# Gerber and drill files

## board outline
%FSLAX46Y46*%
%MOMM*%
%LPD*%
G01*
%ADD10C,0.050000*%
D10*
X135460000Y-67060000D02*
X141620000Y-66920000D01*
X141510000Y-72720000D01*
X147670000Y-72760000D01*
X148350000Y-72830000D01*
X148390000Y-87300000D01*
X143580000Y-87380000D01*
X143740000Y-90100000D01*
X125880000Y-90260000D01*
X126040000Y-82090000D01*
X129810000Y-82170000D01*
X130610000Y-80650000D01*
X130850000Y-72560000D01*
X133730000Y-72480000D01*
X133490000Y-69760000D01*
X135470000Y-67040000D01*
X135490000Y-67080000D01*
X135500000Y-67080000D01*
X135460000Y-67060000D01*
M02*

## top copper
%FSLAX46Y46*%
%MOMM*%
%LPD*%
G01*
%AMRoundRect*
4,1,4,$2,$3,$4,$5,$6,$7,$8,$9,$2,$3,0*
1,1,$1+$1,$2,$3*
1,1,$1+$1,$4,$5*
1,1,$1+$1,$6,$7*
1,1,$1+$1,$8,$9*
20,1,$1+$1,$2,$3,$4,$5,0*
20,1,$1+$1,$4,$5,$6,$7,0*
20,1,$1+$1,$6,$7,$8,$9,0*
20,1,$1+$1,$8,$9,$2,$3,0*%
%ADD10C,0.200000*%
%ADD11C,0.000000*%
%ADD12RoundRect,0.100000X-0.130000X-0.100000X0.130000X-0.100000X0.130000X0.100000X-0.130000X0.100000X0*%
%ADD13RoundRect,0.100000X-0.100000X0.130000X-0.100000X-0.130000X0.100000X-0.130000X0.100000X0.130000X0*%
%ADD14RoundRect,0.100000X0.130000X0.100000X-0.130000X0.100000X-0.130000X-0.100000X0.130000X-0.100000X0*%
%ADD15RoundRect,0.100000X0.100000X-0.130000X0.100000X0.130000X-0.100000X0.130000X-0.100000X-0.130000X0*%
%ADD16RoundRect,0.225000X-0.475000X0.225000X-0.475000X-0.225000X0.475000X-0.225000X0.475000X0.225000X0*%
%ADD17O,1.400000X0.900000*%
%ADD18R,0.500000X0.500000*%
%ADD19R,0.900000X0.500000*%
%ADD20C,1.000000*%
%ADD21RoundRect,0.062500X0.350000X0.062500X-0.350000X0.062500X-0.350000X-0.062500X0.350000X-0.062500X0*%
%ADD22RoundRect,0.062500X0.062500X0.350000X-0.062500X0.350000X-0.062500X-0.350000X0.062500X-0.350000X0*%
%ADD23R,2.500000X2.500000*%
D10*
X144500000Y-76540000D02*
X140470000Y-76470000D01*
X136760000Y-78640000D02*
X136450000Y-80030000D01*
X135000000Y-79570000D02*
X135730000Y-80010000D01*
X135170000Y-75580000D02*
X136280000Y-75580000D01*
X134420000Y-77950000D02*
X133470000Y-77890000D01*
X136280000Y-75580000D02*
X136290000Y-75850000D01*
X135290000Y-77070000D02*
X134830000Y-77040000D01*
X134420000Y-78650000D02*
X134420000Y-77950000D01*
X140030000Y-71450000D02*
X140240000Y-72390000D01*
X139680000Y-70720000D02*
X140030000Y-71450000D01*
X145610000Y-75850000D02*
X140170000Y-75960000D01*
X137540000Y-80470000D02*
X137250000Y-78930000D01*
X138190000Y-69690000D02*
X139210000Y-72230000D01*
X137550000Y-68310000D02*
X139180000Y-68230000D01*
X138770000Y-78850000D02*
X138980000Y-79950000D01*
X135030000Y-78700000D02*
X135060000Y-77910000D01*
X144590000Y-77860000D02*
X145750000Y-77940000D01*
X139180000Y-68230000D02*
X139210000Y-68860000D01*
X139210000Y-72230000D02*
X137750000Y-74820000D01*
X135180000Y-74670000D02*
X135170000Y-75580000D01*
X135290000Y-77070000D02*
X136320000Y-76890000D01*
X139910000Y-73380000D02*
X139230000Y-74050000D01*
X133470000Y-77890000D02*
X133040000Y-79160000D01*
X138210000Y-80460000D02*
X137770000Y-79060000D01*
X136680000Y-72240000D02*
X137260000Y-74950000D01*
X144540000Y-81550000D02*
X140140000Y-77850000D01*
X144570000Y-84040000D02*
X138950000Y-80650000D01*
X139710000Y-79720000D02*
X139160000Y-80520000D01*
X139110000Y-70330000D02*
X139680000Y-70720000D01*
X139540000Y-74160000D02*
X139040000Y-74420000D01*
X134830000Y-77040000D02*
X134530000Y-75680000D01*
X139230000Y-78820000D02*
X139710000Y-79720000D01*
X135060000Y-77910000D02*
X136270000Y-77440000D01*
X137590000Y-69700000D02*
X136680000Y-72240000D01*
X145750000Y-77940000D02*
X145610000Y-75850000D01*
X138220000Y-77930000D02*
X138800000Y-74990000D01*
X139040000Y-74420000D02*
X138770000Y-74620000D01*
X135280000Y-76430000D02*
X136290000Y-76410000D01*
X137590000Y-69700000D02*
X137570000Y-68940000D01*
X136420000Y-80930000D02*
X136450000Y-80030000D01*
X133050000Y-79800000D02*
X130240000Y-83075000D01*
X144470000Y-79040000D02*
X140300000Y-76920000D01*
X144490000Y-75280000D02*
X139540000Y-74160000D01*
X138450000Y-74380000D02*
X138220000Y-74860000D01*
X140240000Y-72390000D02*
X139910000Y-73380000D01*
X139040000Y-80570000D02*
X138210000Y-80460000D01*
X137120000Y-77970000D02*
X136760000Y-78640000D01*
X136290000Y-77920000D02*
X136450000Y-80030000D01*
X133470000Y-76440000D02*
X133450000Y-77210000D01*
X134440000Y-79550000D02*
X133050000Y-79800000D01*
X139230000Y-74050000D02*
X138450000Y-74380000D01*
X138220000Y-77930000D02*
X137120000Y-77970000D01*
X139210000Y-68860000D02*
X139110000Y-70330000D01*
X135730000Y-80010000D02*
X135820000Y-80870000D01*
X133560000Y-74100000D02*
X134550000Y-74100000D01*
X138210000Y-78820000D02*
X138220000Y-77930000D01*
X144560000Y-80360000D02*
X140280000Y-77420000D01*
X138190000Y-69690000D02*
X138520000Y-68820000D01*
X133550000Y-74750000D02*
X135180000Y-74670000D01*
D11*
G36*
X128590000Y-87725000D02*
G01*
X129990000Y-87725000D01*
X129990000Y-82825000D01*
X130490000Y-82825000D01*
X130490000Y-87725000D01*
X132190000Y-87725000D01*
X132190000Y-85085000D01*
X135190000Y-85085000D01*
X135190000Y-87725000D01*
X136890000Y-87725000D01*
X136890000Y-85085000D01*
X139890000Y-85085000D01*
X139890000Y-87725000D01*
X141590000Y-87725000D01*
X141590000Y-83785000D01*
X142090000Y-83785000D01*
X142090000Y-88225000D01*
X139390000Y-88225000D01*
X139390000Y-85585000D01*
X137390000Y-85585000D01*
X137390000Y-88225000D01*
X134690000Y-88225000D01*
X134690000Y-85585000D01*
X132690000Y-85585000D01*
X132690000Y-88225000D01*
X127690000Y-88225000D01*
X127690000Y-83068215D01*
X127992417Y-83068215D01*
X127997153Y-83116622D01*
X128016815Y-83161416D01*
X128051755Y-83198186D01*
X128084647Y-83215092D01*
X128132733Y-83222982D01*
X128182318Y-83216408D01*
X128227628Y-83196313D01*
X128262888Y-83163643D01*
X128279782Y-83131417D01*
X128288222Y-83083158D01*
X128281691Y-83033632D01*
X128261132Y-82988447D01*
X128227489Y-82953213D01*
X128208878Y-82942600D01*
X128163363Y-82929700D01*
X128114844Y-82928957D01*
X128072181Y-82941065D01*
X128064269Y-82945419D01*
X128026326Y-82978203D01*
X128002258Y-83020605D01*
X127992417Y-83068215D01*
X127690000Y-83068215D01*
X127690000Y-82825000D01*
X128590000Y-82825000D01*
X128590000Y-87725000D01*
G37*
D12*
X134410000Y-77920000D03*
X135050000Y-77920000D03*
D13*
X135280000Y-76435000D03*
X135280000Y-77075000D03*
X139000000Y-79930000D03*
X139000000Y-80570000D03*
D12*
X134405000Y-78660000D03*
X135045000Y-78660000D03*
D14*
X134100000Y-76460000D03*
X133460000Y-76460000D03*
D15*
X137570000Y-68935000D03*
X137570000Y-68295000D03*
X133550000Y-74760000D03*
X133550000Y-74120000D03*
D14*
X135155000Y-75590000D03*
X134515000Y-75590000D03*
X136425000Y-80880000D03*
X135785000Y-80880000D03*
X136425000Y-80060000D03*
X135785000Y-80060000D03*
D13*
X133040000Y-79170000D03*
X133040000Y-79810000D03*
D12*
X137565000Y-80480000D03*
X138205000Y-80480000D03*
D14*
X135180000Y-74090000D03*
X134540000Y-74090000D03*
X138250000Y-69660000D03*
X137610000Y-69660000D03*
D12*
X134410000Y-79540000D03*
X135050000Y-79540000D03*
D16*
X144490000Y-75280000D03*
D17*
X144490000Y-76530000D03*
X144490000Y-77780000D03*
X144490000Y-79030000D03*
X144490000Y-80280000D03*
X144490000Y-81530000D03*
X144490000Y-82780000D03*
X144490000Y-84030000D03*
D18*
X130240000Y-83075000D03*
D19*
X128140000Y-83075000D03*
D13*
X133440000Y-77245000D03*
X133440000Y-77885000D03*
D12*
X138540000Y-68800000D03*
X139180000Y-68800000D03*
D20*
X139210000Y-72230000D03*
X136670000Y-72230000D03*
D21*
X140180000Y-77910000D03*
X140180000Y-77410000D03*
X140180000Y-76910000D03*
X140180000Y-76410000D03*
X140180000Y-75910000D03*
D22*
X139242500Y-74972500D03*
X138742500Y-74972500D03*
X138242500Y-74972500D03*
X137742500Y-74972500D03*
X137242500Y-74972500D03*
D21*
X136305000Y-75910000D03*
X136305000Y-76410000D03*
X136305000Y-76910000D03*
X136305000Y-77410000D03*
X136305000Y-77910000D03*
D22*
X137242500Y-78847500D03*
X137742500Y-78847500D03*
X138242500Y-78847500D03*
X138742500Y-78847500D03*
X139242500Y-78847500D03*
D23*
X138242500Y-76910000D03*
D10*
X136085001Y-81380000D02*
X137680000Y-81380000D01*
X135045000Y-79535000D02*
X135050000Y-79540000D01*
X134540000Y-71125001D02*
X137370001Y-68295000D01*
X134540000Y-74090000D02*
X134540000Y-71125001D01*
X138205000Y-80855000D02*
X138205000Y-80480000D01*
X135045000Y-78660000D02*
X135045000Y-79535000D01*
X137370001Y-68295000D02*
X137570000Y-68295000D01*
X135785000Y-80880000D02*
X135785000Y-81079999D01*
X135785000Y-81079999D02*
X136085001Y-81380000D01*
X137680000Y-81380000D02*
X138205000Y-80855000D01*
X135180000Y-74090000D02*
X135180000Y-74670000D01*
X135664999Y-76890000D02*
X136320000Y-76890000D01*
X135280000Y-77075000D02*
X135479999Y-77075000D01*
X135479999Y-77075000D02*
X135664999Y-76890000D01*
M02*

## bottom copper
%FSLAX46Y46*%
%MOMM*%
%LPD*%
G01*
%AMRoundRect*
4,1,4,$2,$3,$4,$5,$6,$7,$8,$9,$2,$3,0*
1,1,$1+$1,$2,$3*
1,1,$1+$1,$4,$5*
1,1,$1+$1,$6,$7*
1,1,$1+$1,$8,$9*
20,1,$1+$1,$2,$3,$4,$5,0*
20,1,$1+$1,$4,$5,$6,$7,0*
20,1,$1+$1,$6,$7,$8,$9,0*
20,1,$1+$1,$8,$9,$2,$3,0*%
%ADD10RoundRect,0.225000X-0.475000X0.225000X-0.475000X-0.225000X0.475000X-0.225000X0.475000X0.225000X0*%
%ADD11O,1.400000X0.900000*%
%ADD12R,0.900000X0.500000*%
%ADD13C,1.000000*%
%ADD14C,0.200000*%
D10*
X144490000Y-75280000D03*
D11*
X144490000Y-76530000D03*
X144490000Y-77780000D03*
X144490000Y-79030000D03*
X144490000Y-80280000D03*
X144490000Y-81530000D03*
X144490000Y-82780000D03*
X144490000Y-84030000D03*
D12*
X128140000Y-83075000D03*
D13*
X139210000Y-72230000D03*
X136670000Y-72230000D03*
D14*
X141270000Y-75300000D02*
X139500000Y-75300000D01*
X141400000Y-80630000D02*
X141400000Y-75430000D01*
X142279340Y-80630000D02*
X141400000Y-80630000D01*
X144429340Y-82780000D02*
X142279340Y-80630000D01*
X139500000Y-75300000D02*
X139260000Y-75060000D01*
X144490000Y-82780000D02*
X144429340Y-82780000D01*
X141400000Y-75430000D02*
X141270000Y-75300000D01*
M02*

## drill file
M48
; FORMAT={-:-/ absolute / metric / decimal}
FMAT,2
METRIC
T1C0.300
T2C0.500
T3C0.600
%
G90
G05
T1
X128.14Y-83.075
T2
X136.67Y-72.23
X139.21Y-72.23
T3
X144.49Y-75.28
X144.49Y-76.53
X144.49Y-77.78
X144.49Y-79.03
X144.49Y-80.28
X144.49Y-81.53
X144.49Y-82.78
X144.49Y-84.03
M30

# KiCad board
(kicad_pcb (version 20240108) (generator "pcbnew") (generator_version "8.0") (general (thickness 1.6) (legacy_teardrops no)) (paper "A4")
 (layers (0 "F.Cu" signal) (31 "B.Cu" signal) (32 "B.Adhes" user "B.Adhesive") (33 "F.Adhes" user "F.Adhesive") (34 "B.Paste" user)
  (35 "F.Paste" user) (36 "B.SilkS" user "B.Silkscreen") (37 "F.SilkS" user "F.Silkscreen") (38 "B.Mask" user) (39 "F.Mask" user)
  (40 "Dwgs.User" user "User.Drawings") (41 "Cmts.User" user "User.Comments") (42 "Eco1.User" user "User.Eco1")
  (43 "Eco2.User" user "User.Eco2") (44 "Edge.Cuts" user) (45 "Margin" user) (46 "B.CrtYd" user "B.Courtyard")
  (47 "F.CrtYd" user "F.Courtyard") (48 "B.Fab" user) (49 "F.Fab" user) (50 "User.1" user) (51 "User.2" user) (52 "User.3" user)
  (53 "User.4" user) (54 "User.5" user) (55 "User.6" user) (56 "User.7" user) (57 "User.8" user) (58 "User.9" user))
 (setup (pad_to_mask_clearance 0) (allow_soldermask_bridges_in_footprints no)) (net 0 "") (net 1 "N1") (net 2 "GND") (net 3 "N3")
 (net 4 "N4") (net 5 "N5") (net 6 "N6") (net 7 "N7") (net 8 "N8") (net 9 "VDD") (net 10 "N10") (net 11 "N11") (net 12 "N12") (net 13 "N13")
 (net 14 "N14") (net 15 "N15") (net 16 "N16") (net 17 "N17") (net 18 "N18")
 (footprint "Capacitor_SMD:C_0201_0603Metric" (layer "F.Cu") (at 134.73 77.92)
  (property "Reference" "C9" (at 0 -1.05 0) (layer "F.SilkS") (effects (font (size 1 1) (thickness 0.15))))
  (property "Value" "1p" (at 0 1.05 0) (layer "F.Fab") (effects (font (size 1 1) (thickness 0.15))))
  (pad "" smd roundrect (at -0.345 0) (size 0.318 0.36) (layers "F.Paste") (roundrect_rratio 0.25))
  (pad "" smd roundrect (at 0.345 0) (size 0.318 0.36) (layers "F.Paste") (roundrect_rratio 0.25))
  (pad "1" smd roundrect (at -0.32 0) (size 0.46 0.4) (layers "F.Cu" "F.Mask") (roundrect_rratio 0.25) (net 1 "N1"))
  (pad "2" smd roundrect (at 0.32 0) (size 0.46 0.4) (layers "F.Cu" "F.Mask") (roundrect_rratio 0.25) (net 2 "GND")))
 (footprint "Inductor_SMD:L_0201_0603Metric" (layer "F.Cu") (at 135.28 76.755 -90)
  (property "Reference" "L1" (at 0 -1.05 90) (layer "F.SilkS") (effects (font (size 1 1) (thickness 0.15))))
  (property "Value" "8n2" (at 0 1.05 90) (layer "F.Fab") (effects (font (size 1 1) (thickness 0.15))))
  (pad "" smd roundrect (at -0.345 0 270) (size 0.318 0.36) (layers "F.Paste") (roundrect_rratio 0.25))
  (pad "" smd roundrect (at 0.345 0 270) (size 0.318 0.36) (layers "F.Paste") (roundrect_rratio 0.25))
  (pad "1" smd roundrect (at -0.32 0 270) (size 0.46 0.4) (layers "F.Cu" "F.Mask") (roundrect_rratio 0.25) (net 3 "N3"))
  (pad "2" smd roundrect (at 0.32 0 270) (size 0.46 0.4) (layers "F.Cu" "F.Mask") (roundrect_rratio 0.25) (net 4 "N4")))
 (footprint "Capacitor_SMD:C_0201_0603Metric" (layer "F.Cu") (at 139 80.25 -90)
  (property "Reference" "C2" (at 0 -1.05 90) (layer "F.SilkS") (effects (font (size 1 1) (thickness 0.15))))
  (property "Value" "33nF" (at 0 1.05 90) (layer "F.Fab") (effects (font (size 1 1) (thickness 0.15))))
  (pad "" smd roundrect (at -0.345 0 270) (size 0.318 0.36) (layers "F.Paste") (roundrect_rratio 0.25))
  (pad "" smd roundrect (at 0.345 0 270) (size 0.318 0.36) (layers "F.Paste") (roundrect_rratio 0.25))
  (pad "1" smd roundrect (at -0.32 0 270) (size 0.46 0.4) (layers "F.Cu" "F.Mask") (roundrect_rratio 0.25) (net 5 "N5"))
  (pad "2" smd roundrect (at 0.32 0 270) (size 0.46 0.4) (layers "F.Cu" "F.Mask") (roundrect_rratio 0.25) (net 2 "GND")))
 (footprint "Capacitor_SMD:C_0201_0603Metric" (layer "F.Cu") (at 134.725 78.66)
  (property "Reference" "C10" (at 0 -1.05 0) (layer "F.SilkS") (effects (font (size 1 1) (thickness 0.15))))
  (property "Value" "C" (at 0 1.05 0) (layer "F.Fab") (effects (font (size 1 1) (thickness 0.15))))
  (pad "" smd roundrect (at -0.345 0) (size 0.318 0.36) (layers "F.Paste") (roundrect_rratio 0.25))
  (pad "" smd roundrect (at 0.345 0) (size 0.318 0.36) (layers "F.Paste") (roundrect_rratio 0.25))
  (pad "1" smd roundrect (at -0.32 0) (size 0.46 0.4) (layers "F.Cu" "F.Mask") (roundrect_rratio 0.25) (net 1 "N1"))
  (pad "2" smd roundrect (at 0.32 0) (size 0.46 0.4) (layers "F.Cu" "F.Mask") (roundrect_rratio 0.25) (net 2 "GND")))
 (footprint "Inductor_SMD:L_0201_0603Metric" (layer "F.Cu") (at 133.78 76.46 180)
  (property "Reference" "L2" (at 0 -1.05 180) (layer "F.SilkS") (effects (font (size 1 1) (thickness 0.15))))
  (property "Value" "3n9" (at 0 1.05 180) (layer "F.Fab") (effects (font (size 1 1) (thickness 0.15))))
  (pad "" smd roundrect (at -0.345 0 180) (size 0.318 0.36) (layers "F.Paste") (roundrect_rratio 0.25))
  (pad "" smd roundrect (at 0.345 0 180) (size 0.318 0.36) (layers "F.Paste") (roundrect_rratio 0.25))
  (pad "1" smd roundrect (at -0.32 0 180) (size 0.46 0.4) (layers "F.Cu" "F.Mask") (roundrect_rratio 0.25) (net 3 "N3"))
  (pad "2" smd roundrect (at 0.32 0 180) (size 0.46 0.4) (layers "F.Cu" "F.Mask") (roundrect_rratio 0.25) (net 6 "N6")))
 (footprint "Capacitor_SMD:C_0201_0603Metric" (layer "F.Cu") (at 137.57 68.615 90)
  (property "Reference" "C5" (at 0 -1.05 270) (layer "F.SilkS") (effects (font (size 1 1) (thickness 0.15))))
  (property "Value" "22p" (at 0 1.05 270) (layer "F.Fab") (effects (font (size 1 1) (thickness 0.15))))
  (pad "" smd roundrect (at -0.345 0 90) (size 0.318 0.36) (layers "F.Paste") (roundrect_rratio 0.25))
  (pad "" smd roundrect (at 0.345 0 90) (size 0.318 0.36) (layers "F.Paste") (roundrect_rratio 0.25))
  (pad "1" smd roundrect (at -0.32 0 90) (size 0.46 0.4) (layers "F.Cu" "F.Mask") (roundrect_rratio 0.25) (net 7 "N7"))
  (pad "2" smd roundrect (at 0.32 0 90) (size 0.46 0.4) (layers "F.Cu" "F.Mask") (roundrect_rratio 0.25) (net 2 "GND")))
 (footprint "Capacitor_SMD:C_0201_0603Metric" (layer "F.Cu") (at 133.55 74.44 90)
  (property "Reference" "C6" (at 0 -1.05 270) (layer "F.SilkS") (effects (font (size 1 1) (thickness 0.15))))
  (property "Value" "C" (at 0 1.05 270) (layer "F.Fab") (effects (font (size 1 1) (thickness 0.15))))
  (pad "" smd roundrect (at -0.345 0 90) (size 0.318 0.36) (layers "F.Paste") (roundrect_rratio 0.25))
  (pad "" smd roundrect (at 0.345 0 90) (size 0.318 0.36) (layers "F.Paste") (roundrect_rratio 0.25))
  (pad "1" smd roundrect (at -0.32 0 90) (size 0.46 0.4) (layers "F.Cu" "F.Mask") (roundrect_rratio 0.25) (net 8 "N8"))
  (pad "2" smd roundrect (at 0.32 0 90) (size 0.46 0.4) (layers "F.Cu" "F.Mask") (roundrect_rratio 0.25) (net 2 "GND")))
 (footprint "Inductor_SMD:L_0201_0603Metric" (layer "F.Cu") (at 134.835 75.59 180)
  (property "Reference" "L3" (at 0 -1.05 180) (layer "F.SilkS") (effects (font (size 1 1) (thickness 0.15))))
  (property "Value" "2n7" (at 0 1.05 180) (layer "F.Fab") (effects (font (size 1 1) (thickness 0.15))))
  (pad "" smd roundrect (at -0.345 0 180) (size 0.318 0.36) (layers "F.Paste") (roundrect_rratio 0.25))
  (pad "" smd roundrect (at 0.345 0 180) (size 0.318 0.36) (layers "F.Paste") (roundrect_rratio 0.25))
  (pad "1" smd roundrect (at -0.32 0 180) (size 0.46 0.4) (layers "F.Cu" "F.Mask") (roundrect_rratio 0.25) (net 8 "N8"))
  (pad "2" smd roundrect (at 0.32 0 180) (size 0.46 0.4) (layers "F.Cu" "F.Mask") (roundrect_rratio 0.25) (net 4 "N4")))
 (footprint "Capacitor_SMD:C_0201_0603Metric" (layer "F.Cu") (at 136.105 80.88 180)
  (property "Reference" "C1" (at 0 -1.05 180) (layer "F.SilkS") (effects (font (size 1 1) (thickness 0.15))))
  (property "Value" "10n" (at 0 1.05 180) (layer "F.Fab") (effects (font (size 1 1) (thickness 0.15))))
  (pad "" smd roundrect (at -0.345 0 180) (size 0.318 0.36) (layers "F.Paste") (roundrect_rratio 0.25))
  (pad "" smd roundrect (at 0.345 0 180) (size 0.318 0.36) (layers "F.Paste") (roundrect_rratio 0.25))
  (pad "1" smd roundrect (at -0.32 0 180) (size 0.46 0.4) (layers "F.Cu" "F.Mask") (roundrect_rratio 0.25) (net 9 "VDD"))
  (pad "2" smd roundrect (at 0.32 0 180) (size 0.46 0.4) (layers "F.Cu" "F.Mask") (roundrect_rratio 0.25) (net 2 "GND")))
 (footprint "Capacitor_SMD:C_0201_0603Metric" (layer "F.Cu") (at 136.105 80.06 180)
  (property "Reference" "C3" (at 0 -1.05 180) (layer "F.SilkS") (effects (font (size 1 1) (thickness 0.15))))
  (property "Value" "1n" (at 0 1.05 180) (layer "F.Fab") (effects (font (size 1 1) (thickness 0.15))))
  (pad "" smd roundrect (at -0.345 0 180) (size 0.318 0.36) (layers "F.Paste") (roundrect_rratio 0.25))
  (pad "" smd roundrect (at 0.345 0 180) (size 0.318 0.36) (layers "F.Paste") (roundrect_rratio 0.25))
  (pad "1" smd roundrect (at -0.32 0 180) (size 0.46 0.4) (layers "F.Cu" "F.Mask") (roundrect_rratio 0.25) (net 9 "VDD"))
  (pad "2" smd roundrect (at 0.32 0 180) (size 0.46 0.4) (layers "F.Cu" "F.Mask") (roundrect_rratio 0.25) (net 2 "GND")))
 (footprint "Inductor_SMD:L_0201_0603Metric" (layer "F.Cu") (at 133.04 79.49 -90)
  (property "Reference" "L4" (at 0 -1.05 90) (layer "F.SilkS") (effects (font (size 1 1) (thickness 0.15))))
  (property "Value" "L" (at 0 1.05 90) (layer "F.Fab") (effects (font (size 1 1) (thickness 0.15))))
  (pad "" smd roundrect (at -0.345 0 270) (size 0.318 0.36) (layers "F.Paste") (roundrect_rratio 0.25))
  (pad "" smd roundrect (at 0.345 0 270) (size 0.318 0.36) (layers "F.Paste") (roundrect_rratio 0.25))
  (pad "1" smd roundrect (at -0.32 0 270) (size 0.46 0.4) (layers "F.Cu" "F.Mask") (roundrect_rratio 0.25) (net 1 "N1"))
  (pad "2" smd roundrect (at 0.32 0 270) (size 0.46 0.4) (layers "F.Cu" "F.Mask") (roundrect_rratio 0.25) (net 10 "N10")))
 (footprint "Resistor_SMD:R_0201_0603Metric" (layer "F.Cu") (at 137.885 80.48)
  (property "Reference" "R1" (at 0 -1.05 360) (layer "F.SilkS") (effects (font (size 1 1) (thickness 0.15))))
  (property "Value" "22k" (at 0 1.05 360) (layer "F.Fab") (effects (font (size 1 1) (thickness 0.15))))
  (pad "" smd roundrect (at -0.345 0) (size 0.318 0.36) (layers "F.Paste") (roundrect_rratio 0.25))
  (pad "" smd roundrect (at 0.345 0) (size 0.318 0.36) (layers "F.Paste") (roundrect_rratio 0.25))
  (pad "1" smd roundrect (at -0.32 0) (size 0.46 0.4) (layers "F.Cu" "F.Mask") (roundrect_rratio 0.25) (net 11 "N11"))
  (pad "2" smd roundrect (at 0.32 0) (size 0.46 0.4) (layers "F.Cu" "F.Mask") (roundrect_rratio 0.25) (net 2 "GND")))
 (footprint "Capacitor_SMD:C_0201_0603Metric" (layer "F.Cu") (at 134.86 74.09 180)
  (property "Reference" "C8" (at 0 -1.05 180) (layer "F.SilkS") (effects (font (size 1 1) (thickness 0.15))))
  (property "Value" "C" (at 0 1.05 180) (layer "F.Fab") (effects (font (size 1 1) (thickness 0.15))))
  (pad "" smd roundrect (at -0.345 0 180) (size 0.318 0.36) (layers "F.Paste") (roundrect_rratio 0.25))
  (pad "" smd roundrect (at 0.345 0 180) (size 0.318 0.36) (layers "F.Paste") (roundrect_rratio 0.25))
  (pad "1" smd roundrect (at -0.32 0 180) (size 0.46 0.4) (layers "F.Cu" "F.Mask") (roundrect_rratio 0.25) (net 8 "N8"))
  (pad "2" smd roundrect (at 0.32 0 180) (size 0.46 0.4) (layers "F.Cu" "F.Mask") (roundrect_rratio 0.25) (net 2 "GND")))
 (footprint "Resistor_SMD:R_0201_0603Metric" (layer "F.Cu") (at 137.93 69.66 180)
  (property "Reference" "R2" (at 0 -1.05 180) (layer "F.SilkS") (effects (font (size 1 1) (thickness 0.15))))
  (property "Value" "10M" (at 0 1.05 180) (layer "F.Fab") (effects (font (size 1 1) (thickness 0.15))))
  (pad "" smd roundrect (at -0.345 0 180) (size 0.318 0.36) (layers "F.Paste") (roundrect_rratio 0.25))
  (pad "" smd roundrect (at 0.345 0 180) (size 0.318 0.36) (layers "F.Paste") (roundrect_rratio 0.25))
  (pad "1" smd roundrect (at -0.32 0 180) (size 0.46 0.4) (layers "F.Cu" "F.Mask") (roundrect_rratio 0.25) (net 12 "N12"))
  (pad "2" smd roundrect (at 0.32 0 180) (size 0.46 0.4) (layers "F.Cu" "F.Mask") (roundrect_rratio 0.25) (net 7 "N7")))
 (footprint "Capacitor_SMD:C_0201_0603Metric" (layer "F.Cu") (at 134.73 79.54)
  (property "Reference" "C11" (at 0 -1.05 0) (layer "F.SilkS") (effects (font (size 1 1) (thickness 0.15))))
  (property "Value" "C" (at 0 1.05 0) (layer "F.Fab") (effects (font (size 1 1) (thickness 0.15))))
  (pad "" smd roundrect (at -0.345 0) (size 0.318 0.36) (layers "F.Paste") (roundrect_rratio 0.25))
  (pad "" smd roundrect (at 0.345 0) (size 0.318 0.36) (layers "F.Paste") (roundrect_rratio 0.25))
  (pad "1" smd roundrect (at -0.32 0) (size 0.46 0.4) (layers "F.Cu" "F.Mask") (roundrect_rratio 0.25) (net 10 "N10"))
  (pad "2" smd roundrect (at 0.32 0) (size 0.46 0.4) (layers "F.Cu" "F.Mask") (roundrect_rratio 0.25) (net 2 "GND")))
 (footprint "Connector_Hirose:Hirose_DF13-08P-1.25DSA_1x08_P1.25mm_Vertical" (layer "F.Cu") (at 144.49 75.28 -90)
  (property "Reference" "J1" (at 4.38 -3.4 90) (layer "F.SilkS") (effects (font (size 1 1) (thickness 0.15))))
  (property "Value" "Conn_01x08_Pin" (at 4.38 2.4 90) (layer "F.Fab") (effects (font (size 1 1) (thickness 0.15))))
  (pad "1" thru_hole roundrect (at 0 0 270) (size 0.9 1.4) (drill 0.6) (layers "*.Cu" "*.Mask") (remove_unused_layers no)
   (roundrect_rratio 0.25) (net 9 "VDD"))
  (pad "2" thru_hole oval (at 1.25 0 270) (size 0.9 1.4) (drill 0.6) (layers "*.Cu" "*.Mask") (remove_unused_layers no) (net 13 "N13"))
  (pad "3" thru_hole oval (at 2.5 0 270) (size 0.9 1.4) (drill 0.6) (layers "*.Cu" "*.Mask") (remove_unused_layers no) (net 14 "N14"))
  (pad "4" thru_hole oval (at 3.75 0 270) (size 0.9 1.4) (drill 0.6) (layers "*.Cu" "*.Mask") (remove_unused_layers no) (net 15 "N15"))
  (pad "5" thru_hole oval (at 5 0 270) (size 0.9 1.4) (drill 0.6) (layers "*.Cu" "*.Mask") (remove_unused_layers no) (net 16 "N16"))
  (pad "6" thru_hole oval (at 6.25 0 270) (size 0.9 1.4) (drill 0.6) (layers "*.Cu" "*.Mask") (remove_unused_layers no) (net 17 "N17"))
  (pad "7" thru_hole oval (at 7.5 0 270) (size 0.9 1.4) (drill 0.6) (layers "*.Cu" "*.Mask") (remove_unused_layers no) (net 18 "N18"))
  (pad "8" thru_hole oval (at 8.75 0 270) (size 0.9 1.4) (drill 0.6) (layers "*.Cu" "*.Mask") (remove_unused_layers no) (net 2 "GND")))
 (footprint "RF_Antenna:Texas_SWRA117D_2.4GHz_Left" (layer "F.Cu") (at 130.24 83.075 180)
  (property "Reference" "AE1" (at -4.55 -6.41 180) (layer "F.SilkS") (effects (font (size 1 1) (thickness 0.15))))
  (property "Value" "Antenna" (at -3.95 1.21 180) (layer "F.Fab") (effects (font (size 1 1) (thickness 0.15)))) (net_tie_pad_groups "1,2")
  (fp_poly
   (pts (xy -2.45 -2.51) (xy -4.45 -2.51) (xy -4.45 -5.15) (xy -7.15 -5.15) (xy -7.15 -2.51) (xy -9.15 -2.51) (xy -9.15 -5.15)
    (xy -11.85 -5.15) (xy -11.85 -0.71) (xy -11.35 -0.71) (xy -11.35 -4.65) (xy -9.65 -4.65) (xy -9.65 -2.01) (xy -6.65 -2.01)
    (xy -6.65 -4.65) (xy -4.95 -4.65) (xy -4.95 -2.01) (xy -1.95 -2.01) (xy -1.95 -4.65) (xy -0.25 -4.65) (xy -0.25 0.25) (xy 0.25 0.25)
    (xy 0.25 -4.65) (xy 1.65 -4.65) (xy 1.65 0.25) (xy 2.55 0.25) (xy 2.55 0.006785) (xy 2.247583 0.006785) (xy 2.237742 0.054395)
    (xy 2.213674 0.096797) (xy 2.175731 0.129581) (xy 2.167819 0.133935) (xy 2.125156 0.146043) (xy 2.076637 0.1453) (xy 2.031122 0.1324)
    (xy 2.012511 0.121787) (xy 1.978868 0.086553) (xy 1.958309 0.041368) (xy 1.951778 -0.008158) (xy 1.960218 -0.056417)
    (xy 1.977112 -0.088643) (xy 2.012372 -0.121313) (xy 2.057682 -0.141408) (xy 2.107267 -0.147982) (xy 2.155353 -0.140092)
    (xy 2.188245 -0.123186) (xy 2.223185 -0.086416) (xy 2.242847 -0.041622) (xy 2.247583 0.006785) (xy 2.55 0.006785) (xy 2.55 -5.15)
    (xy -2.45 -5.15) (xy -2.45 -2.51))
   (stroke (width 0) (type solid)) (fill solid) (layer "F.Cu"))
  (pad "1" connect rect (at 0 0 180) (size 0.5 0.5) (layers "F.Cu") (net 10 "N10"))
  (pad "2" thru_hole rect (at 2.1 0 180) (size 0.9 0.5) (drill 0.3) (layers "*.Cu") (remove_unused_layers no) (zone_connect 2)))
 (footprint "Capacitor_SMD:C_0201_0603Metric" (layer "F.Cu") (at 133.44 77.565 -90)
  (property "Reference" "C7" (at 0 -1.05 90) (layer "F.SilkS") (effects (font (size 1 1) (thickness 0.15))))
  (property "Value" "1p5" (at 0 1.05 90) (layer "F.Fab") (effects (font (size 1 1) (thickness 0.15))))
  (pad "" smd roundrect (at -0.345 0 270) (size 0.318 0.36) (layers "F.Paste") (roundrect_rratio 0.25))
  (pad "" smd roundrect (at 0.345 0 270) (size 0.318 0.36) (layers "F.Paste") (roundrect_rratio 0.25))
  (pad "1" smd roundrect (at -0.32 0 270) (size 0.46 0.4) (layers "F.Cu" "F.Mask") (roundrect_rratio 0.25) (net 6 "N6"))
  (pad "2" smd roundrect (at 0.32 0 270) (size 0.46 0.4) (layers "F.Cu" "F.Mask") (roundrect_rratio 0.25) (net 1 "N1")))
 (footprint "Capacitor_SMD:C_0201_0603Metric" (layer "F.Cu") (at 138.86 68.8)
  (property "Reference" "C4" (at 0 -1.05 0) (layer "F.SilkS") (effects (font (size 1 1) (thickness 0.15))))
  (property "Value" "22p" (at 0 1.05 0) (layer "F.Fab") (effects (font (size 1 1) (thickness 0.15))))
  (pad "" smd roundrect (at -0.345 0) (size 0.318 0.36) (layers "F.Paste") (roundrect_rratio 0.25))
  (pad "" smd roundrect (at 0.345 0) (size 0.318 0.36) (layers "F.Paste") (roundrect_rratio 0.25))
  (pad "1" smd roundrect (at -0.32 0) (size 0.46 0.4) (layers "F.Cu" "F.Mask") (roundrect_rratio 0.25) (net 12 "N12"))
  (pad "2" smd roundrect (at 0.32 0) (size 0.46 0.4) (layers "F.Cu" "F.Mask") (roundrect_rratio 0.25) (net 2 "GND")))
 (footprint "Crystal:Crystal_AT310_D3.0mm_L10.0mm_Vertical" (layer "F.Cu") (at 139.21 72.23 180)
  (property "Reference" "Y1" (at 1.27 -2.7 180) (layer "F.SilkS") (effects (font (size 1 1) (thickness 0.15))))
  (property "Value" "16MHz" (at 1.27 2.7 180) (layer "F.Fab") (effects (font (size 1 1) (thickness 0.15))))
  (pad "1" thru_hole circle (at 0 0 180) (size 1 1) (drill 0.5) (layers "*.Cu" "*.Mask") (remove_unused_layers no) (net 12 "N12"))
  (pad "2" thru_hole circle (at 2.54 0 180) (size 1 1) (drill 0.5) (layers "*.Cu" "*.Mask") (remove_unused_layers no) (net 7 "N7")))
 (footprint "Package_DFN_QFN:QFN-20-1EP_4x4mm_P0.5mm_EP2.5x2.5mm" (layer "F.Cu") (at 138.2425 76.91 180)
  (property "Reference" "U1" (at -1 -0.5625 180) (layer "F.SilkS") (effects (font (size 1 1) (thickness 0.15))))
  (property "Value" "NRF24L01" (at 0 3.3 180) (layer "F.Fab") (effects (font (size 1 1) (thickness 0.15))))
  (pad "" smd roundrect (at -0.625 -0.625 180) (size 1.01 1.01) (layers "F.Paste") (roundrect_rratio 0.247525))
  (pad "" smd roundrect (at -0.625 0.625 180) (size 1.01 1.01) (layers "F.Paste") (roundrect_rratio 0.247525))
  (pad "" smd roundrect (at 0.625 -0.625 180) (size 1.01 1.01) (layers "F.Paste") (roundrect_rratio 0.247525))
  (pad "" smd roundrect (at 0.625 0.625 180) (size 1.01 1.01) (layers "F.Paste") (roundrect_rratio 0.247525))
  (pad "1" smd roundrect (at -1.9375 -1 180) (size 0.825 0.25) (layers "F.Cu" "F.Paste" "F.Mask") (roundrect_rratio 0.25) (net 17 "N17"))
  (pad "2" smd roundrect (at -1.9375 -0.5 180) (size 0.825 0.25) (layers "F.Cu" "F.Paste" "F.Mask") (roundrect_rratio 0.25) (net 16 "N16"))
  (pad "3" smd roundrect (at -1.9375 0 180) (size 0.825 0.25) (layers "F.Cu" "F.Paste" "F.Mask") (roundrect_rratio 0.25) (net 15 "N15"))
  (pad "4" smd roundrect (at -1.9375 0.5 180) (size 0.825 0.25) (layers "F.Cu" "F.Paste" "F.Mask") (roundrect_rratio 0.25) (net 13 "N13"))
  (pad "5" smd roundrect (at -1.9375 1 180) (size 0.825 0.25) (layers "F.Cu" "F.Paste" "F.Mask") (roundrect_rratio 0.25) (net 14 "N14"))
  (pad "6" smd roundrect (at -1 1.9375 180) (size 0.25 0.825) (layers "F.Cu" "F.Paste" "F.Mask") (roundrect_rratio 0.25) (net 18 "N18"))
  (pad "7" smd roundrect (at -0.5 1.9375 180) (size 0.25 0.825) (layers "F.Cu" "F.Paste" "F.Mask") (roundrect_rratio 0.25) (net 9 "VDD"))
  (pad "8" smd roundrect (at 0 1.9375 180) (size 0.25 0.825) (layers "F.Cu" "F.Paste" "F.Mask") (roundrect_rratio 0.25) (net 2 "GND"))
  (pad "9" smd roundrect (at 0.5 1.9375 180) (size 0.25 0.825) (layers "F.Cu" "F.Paste" "F.Mask") (roundrect_rratio 0.25) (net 12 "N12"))
  (pad "10" smd roundrect (at 1 1.9375 180) (size 0.25 0.825) (layers "F.Cu" "F.Paste" "F.Mask") (roundrect_rratio 0.25) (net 7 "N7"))
  (pad "11" smd roundrect (at 1.9375 1 180) (size 0.825 0.25) (layers "F.Cu" "F.Paste" "F.Mask") (roundrect_rratio 0.25) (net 8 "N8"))
  (pad "12" smd roundrect (at 1.9375 0.5 180) (size 0.825 0.25) (layers "F.Cu" "F.Paste" "F.Mask") (roundrect_rratio 0.25) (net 3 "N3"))
  (pad "13" smd roundrect (at 1.9375 0 180) (size 0.825 0.25) (layers "F.Cu" "F.Paste" "F.Mask") (roundrect_rratio 0.25) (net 4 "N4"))
  (pad "14" smd roundrect (at 1.9375 -0.5 180) (size 0.825 0.25) (layers "F.Cu" "F.Paste" "F.Mask") (roundrect_rratio 0.25) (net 2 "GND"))
  (pad "15" smd roundrect (at 1.9375 -1 180) (size 0.825 0.25) (layers "F.Cu" "F.Paste" "F.Mask") (roundrect_rratio 0.25) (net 9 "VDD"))
  (pad "16" smd roundrect (at 1 -1.9375 180) (size 0.25 0.825) (layers "F.Cu" "F.Paste" "F.Mask") (roundrect_rratio 0.25) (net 11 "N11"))
  (pad "17" smd roundrect (at 0.5 -1.9375 180) (size 0.25 0.825) (layers "F.Cu" "F.Paste" "F.Mask") (roundrect_rratio 0.25) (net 2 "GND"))
  (pad "18" smd roundrect (at 0 -1.9375 180) (size 0.25 0.825) (layers "F.Cu" "F.Paste" "F.Mask") (roundrect_rratio 0.25) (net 9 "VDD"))
  (pad "19" smd roundrect (at -0.5 -1.9375 180) (size 0.25 0.825) (layers "F.Cu" "F.Paste" "F.Mask") (roundrect_rratio 0.25) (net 5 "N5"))
  (pad "20" smd roundrect (at -1 -1.9375 180) (size 0.25 0.825) (layers "F.Cu" "F.Paste" "F.Mask") (roundrect_rratio 0.25) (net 2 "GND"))
  (pad "21" smd rect (at 0 0 180) (size 2.5 2.5) (layers "F.Cu" "F.Mask") (zone_connect 2)))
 (gr_line (start 144.5 76.54) (end 140.47 76.47) (stroke (width 0.2) (type default)) (layer "F.Cu") (net 13))
 (gr_line (start 136.76 78.64) (end 136.45 80.03) (stroke (width 0.2) (type default)) (layer "F.Cu") (net 9))
 (gr_line (start 135 79.57) (end 135.73 80.01) (stroke (width 0.2) (type default)) (layer "F.Cu") (net 2))
 (gr_line (start 135.17 75.58) (end 136.28 75.58) (stroke (width 0.2) (type default)) (layer "F.Cu") (net 8))
 (gr_line (start 134.42 77.95) (end 133.47 77.89) (stroke (width 0.2) (type default)) (layer "F.Cu") (net 1))
 (gr_line (start 136.28 75.58) (end 136.29 75.85) (stroke (width 0.2) (type default)) (layer "F.Cu") (net 8))
 (gr_line (start 135.29 77.07) (end 134.83 77.04) (stroke (width 0.2) (type default)) (layer "F.Cu") (net 4))
 (gr_line (start 134.42 78.65) (end 134.42 77.95) (stroke (width 0.2) (type default)) (layer "F.Cu") (net 1))
 (gr_line (start 140.03 71.45) (end 140.24 72.39) (stroke (width 0.2) (type default)) (layer "F.Cu") (net 2))
 (gr_line (start 139.68 70.72) (end 140.03 71.45) (stroke (width 0.2) (type default)) (layer "F.Cu") (net 2))
 (gr_line (start 145.61 75.85) (end 140.17 75.96) (stroke (width 0.2) (type default)) (layer "F.Cu") (net 14))
 (gr_line (start 137.54 80.47) (end 137.25 78.93) (stroke (width 0.2) (type default)) (layer "F.Cu") (net 11))
 (gr_line (start 138.19 69.69) (end 139.21 72.23) (stroke (width 0.2) (type default)) (layer "F.Cu") (net 12))
 (gr_line (start 137.55 68.31) (end 139.18 68.23) (stroke (width 0.2) (type default)) (layer "F.Cu") (net 2))
 (gr_line (start 138.77 78.85) (end 138.98 79.95) (stroke (width 0.2) (type default)) (layer "F.Cu") (net 5))
 (gr_line (start 135.03 78.7) (end 135.06 77.91) (stroke (width 0.2) (type default)) (layer "F.Cu") (net 2))
 (gr_line (start 144.59 77.86) (end 145.75 77.94) (stroke (width 0.2) (type default)) (layer "F.Cu") (net 14))
 (gr_line (start 139.18 68.23) (end 139.21 68.86) (stroke (width 0.2) (type default)) (layer "F.Cu") (net 2))
 (gr_line (start 139.21 72.23) (end 137.75 74.82) (stroke (width 0.2) (type default)) (layer "F.Cu") (net 12))
 (gr_line (start 135.18 74.67) (end 135.17 75.58) (stroke (width 0.2) (type default)) (layer "F.Cu") (net 8))
 (gr_line (start 135.29 77.07) (end 136.32 76.89) (stroke (width 0.2) (type default)) (layer "F.Cu") (net 4))
 (gr_line (start 139.91 73.38) (end 139.23 74.05) (stroke (width 0.2) (type default)) (layer "F.Cu") (net 2))
 (gr_line (start 133.47 77.89) (end 133.04 79.16) (stroke (width 0.2) (type default)) (layer "F.Cu") (net 1))
 (gr_line (start 138.21 80.46) (end 137.77 79.06) (stroke (width 0.2) (type default)) (layer "F.Cu") (net 2))
 (gr_line (start 136.68 72.24) (end 137.26 74.95) (stroke (width 0.2) (type default)) (layer "F.Cu") (net 7))
 (gr_line (start 144.54 81.55) (end 140.14 77.85) (stroke (width 0.2) (type default)) (layer "F.Cu") (net 17))
 (gr_line (start 144.57 84.04) (end 138.95 80.65) (stroke (width 0.2) (type default)) (layer "F.Cu") (net 2))
 (gr_line (start 139.71 79.72) (end 139.16 80.52) (stroke (width 0.2) (type default)) (layer "F.Cu") (net 2))
 (gr_line (start 139.11 70.33) (end 139.68 70.72) (stroke (width 0.2) (type default)) (layer "F.Cu") (net 2))
 (gr_line (start 139.54 74.16) (end 139.04 74.42) (stroke (width 0.2) (type default)) (layer "F.Cu") (net 9))
 (gr_line (start 134.83 77.04) (end 134.53 75.68) (stroke (width 0.2) (type default)) (layer "F.Cu") (net 4))
 (gr_line (start 139.23 78.82) (end 139.71 79.72) (stroke (width 0.2) (type default)) (layer "F.Cu") (net 2))
 (gr_line (start 135.06 77.91) (end 136.27 77.44) (stroke (width 0.2) (type default)) (layer "F.Cu") (net 2))
 (gr_line (start 137.59 69.7) (end 136.68 72.24) (stroke (width 0.2) (type default)) (layer "F.Cu") (net 7))
 (gr_line (start 145.75 77.94) (end 145.61 75.85) (stroke (width 0.2) (type default)) (layer "F.Cu") (net 14))
 (gr_line (start 138.22 77.93) (end 138.8 74.99) (stroke (width 0.2) (type default)) (layer "F.Cu") (net 9))
 (gr_line (start 139.04 74.42) (end 138.77 74.62) (stroke (width 0.2) (type default)) (layer "F.Cu") (net 9))
 (gr_line (start 135.28 76.43) (end 136.29 76.41) (stroke (width 0.2) (type default)) (layer "F.Cu") (net 3))
 (gr_line (start 137.59 69.7) (end 137.57 68.94) (stroke (width 0.2) (type default)) (layer "F.Cu") (net 7))
 (gr_line (start 136.42 80.93) (end 136.45 80.03) (stroke (width 0.2) (type default)) (layer "F.Cu") (net 9))
 (gr_line (start 133.05 79.8) (end 130.24 83.075) (stroke (width 0.2) (type default)) (layer "F.Cu") (net 10))
 (gr_line (start 144.47 79.04) (end 140.3 76.92) (stroke (width 0.2) (type default)) (layer "F.Cu") (net 15))
 (gr_line (start 144.49 75.28) (end 139.54 74.16) (stroke (width 0.2) (type default)) (layer "F.Cu") (net 9))
 (gr_line (start 138.45 74.38) (end 138.22 74.86) (stroke (width 0.2) (type default)) (layer "F.Cu") (net 2))
 (gr_line (start 140.24 72.39) (end 139.91 73.38) (stroke (width 0.2) (type default)) (layer "F.Cu") (net 2))
 (gr_line (start 139.04 80.57) (end 138.21 80.46) (stroke (width 0.2) (type default)) (layer "F.Cu") (net 2))
 (gr_line (start 137.12 77.97) (end 136.76 78.64) (stroke (width 0.2) (type default)) (layer "F.Cu") (net 9))
 (gr_line (start 136.29 77.92) (end 136.45 80.03) (stroke (width 0.2) (type default)) (layer "F.Cu") (net 9))
 (gr_line (start 133.47 76.44) (end 133.45 77.21) (stroke (width 0.2) (type default)) (layer "F.Cu") (net 6))
 (gr_line (start 134.44 79.55) (end 133.05 79.8) (stroke (width 0.2) (type default)) (layer "F.Cu") (net 10))
 (gr_line (start 139.23 74.05) (end 138.45 74.38) (stroke (width 0.2) (type default)) (layer "F.Cu") (net 2))
 (gr_line (start 138.22 77.93) (end 137.12 77.97) (stroke (width 0.2) (type default)) (layer "F.Cu") (net 9))
 (gr_line (start 139.21 68.86) (end 139.11 70.33) (stroke (width 0.2) (type default)) (layer "F.Cu") (net 2))
 (gr_line (start 135.73 80.01) (end 135.82 80.87) (stroke (width 0.2) (type default)) (layer "F.Cu") (net 2))
 (gr_line (start 133.56 74.1) (end 134.55 74.1) (stroke (width 0.2) (type default)) (layer "F.Cu") (net 2))
 (gr_line (start 138.21 78.82) (end 138.22 77.93) (stroke (width 0.2) (type default)) (layer "F.Cu") (net 9))
 (gr_line (start 144.56 80.36) (end 140.28 77.42) (stroke (width 0.2) (type default)) (layer "F.Cu") (net 16))
 (gr_line (start 138.19 69.69) (end 138.52 68.82) (stroke (width 0.2) (type default)) (layer "F.Cu") (net 12))
 (gr_line (start 133.55 74.75) (end 135.18 74.67) (stroke (width 0.2) (type default)) (layer "F.Cu") (net 8))
 (gr_poly
  (pts (xy 135.46 67.06) (xy 141.62 66.92) (xy 141.51 72.72) (xy 147.67 72.76) (xy 148.35 72.83) (xy 148.39 87.3) (xy 143.58 87.38)
   (xy 143.74 90.1) (xy 125.88 90.26) (xy 126.04 82.09) (xy 129.81 82.17) (xy 130.61 80.65) (xy 130.85 72.56) (xy 133.73 72.48)
   (xy 133.49 69.76) (xy 135.47 67.04) (xy 135.49 67.08) (xy 135.5 67.08))
  (stroke (width 0.05) (type solid)) (fill none) (layer "Edge.Cuts"))
 (segment (start 136.085001 81.38) (end 137.68 81.38) (width 0.2) (layer "F.Cu") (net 2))
 (segment (start 135.045 79.535) (end 135.05 79.54) (width 0.2) (layer "F.Cu") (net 2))
 (segment (start 134.54 71.125001) (end 137.370001 68.295) (width 0.2) (layer "F.Cu") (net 2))
 (segment (start 134.54 74.09) (end 134.54 71.125001) (width 0.2) (layer "F.Cu") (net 2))
 (segment (start 138.205 80.855) (end 138.205 80.48) (width 0.2) (layer "F.Cu") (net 2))
 (segment (start 135.045 78.66) (end 135.045 79.535) (width 0.2) (layer "F.Cu") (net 2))
 (segment (start 137.370001 68.295) (end 137.57 68.295) (width 0.2) (layer "F.Cu") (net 2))
 (segment (start 135.785 80.88) (end 135.785 81.079999) (width 0.2) (layer "F.Cu") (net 2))
 (segment (start 135.785 81.079999) (end 136.085001 81.38) (width 0.2) (layer "F.Cu") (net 2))
 (segment (start 137.68 81.38) (end 138.205 80.855) (width 0.2) (layer "F.Cu") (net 2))
 (segment (start 135.18 74.09) (end 135.18 74.67) (width 0.2) (layer "F.Cu") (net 8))
 (segment (start 141.27 75.3) (end 139.5 75.3) (width 0.2) (layer "B.Cu") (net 18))
 (segment (start 141.4 80.63) (end 141.4 75.43) (width 0.2) (layer "B.Cu") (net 18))
 (segment (start 142.27934 80.63) (end 141.4 80.63) (width 0.2) (layer "B.Cu") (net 18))
 (segment (start 144.42934 82.78) (end 142.27934 80.63) (width 0.2) (layer "B.Cu") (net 18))
 (segment (start 139.5 75.3) (end 139.26 75.06) (width 0.2) (layer "B.Cu") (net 18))
 (segment (start 144.49 82.78) (end 144.42934 82.78) (width 0.2) (layer "B.Cu") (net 18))
 (segment (start 141.4 75.43) (end 141.27 75.3) (width 0.2) (layer "B.Cu") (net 18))
 (segment (start 135.664999 76.89) (end 136.32 76.89) (width 0.2) (layer "F.Cu") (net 4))
 (segment (start 135.28 77.075) (end 135.479999 77.075) (width 0.2) (layer "F.Cu") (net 4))
 (segment (start 135.479999 77.075) (end 135.664999 76.89) (width 0.2) (layer "F.Cu") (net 4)))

